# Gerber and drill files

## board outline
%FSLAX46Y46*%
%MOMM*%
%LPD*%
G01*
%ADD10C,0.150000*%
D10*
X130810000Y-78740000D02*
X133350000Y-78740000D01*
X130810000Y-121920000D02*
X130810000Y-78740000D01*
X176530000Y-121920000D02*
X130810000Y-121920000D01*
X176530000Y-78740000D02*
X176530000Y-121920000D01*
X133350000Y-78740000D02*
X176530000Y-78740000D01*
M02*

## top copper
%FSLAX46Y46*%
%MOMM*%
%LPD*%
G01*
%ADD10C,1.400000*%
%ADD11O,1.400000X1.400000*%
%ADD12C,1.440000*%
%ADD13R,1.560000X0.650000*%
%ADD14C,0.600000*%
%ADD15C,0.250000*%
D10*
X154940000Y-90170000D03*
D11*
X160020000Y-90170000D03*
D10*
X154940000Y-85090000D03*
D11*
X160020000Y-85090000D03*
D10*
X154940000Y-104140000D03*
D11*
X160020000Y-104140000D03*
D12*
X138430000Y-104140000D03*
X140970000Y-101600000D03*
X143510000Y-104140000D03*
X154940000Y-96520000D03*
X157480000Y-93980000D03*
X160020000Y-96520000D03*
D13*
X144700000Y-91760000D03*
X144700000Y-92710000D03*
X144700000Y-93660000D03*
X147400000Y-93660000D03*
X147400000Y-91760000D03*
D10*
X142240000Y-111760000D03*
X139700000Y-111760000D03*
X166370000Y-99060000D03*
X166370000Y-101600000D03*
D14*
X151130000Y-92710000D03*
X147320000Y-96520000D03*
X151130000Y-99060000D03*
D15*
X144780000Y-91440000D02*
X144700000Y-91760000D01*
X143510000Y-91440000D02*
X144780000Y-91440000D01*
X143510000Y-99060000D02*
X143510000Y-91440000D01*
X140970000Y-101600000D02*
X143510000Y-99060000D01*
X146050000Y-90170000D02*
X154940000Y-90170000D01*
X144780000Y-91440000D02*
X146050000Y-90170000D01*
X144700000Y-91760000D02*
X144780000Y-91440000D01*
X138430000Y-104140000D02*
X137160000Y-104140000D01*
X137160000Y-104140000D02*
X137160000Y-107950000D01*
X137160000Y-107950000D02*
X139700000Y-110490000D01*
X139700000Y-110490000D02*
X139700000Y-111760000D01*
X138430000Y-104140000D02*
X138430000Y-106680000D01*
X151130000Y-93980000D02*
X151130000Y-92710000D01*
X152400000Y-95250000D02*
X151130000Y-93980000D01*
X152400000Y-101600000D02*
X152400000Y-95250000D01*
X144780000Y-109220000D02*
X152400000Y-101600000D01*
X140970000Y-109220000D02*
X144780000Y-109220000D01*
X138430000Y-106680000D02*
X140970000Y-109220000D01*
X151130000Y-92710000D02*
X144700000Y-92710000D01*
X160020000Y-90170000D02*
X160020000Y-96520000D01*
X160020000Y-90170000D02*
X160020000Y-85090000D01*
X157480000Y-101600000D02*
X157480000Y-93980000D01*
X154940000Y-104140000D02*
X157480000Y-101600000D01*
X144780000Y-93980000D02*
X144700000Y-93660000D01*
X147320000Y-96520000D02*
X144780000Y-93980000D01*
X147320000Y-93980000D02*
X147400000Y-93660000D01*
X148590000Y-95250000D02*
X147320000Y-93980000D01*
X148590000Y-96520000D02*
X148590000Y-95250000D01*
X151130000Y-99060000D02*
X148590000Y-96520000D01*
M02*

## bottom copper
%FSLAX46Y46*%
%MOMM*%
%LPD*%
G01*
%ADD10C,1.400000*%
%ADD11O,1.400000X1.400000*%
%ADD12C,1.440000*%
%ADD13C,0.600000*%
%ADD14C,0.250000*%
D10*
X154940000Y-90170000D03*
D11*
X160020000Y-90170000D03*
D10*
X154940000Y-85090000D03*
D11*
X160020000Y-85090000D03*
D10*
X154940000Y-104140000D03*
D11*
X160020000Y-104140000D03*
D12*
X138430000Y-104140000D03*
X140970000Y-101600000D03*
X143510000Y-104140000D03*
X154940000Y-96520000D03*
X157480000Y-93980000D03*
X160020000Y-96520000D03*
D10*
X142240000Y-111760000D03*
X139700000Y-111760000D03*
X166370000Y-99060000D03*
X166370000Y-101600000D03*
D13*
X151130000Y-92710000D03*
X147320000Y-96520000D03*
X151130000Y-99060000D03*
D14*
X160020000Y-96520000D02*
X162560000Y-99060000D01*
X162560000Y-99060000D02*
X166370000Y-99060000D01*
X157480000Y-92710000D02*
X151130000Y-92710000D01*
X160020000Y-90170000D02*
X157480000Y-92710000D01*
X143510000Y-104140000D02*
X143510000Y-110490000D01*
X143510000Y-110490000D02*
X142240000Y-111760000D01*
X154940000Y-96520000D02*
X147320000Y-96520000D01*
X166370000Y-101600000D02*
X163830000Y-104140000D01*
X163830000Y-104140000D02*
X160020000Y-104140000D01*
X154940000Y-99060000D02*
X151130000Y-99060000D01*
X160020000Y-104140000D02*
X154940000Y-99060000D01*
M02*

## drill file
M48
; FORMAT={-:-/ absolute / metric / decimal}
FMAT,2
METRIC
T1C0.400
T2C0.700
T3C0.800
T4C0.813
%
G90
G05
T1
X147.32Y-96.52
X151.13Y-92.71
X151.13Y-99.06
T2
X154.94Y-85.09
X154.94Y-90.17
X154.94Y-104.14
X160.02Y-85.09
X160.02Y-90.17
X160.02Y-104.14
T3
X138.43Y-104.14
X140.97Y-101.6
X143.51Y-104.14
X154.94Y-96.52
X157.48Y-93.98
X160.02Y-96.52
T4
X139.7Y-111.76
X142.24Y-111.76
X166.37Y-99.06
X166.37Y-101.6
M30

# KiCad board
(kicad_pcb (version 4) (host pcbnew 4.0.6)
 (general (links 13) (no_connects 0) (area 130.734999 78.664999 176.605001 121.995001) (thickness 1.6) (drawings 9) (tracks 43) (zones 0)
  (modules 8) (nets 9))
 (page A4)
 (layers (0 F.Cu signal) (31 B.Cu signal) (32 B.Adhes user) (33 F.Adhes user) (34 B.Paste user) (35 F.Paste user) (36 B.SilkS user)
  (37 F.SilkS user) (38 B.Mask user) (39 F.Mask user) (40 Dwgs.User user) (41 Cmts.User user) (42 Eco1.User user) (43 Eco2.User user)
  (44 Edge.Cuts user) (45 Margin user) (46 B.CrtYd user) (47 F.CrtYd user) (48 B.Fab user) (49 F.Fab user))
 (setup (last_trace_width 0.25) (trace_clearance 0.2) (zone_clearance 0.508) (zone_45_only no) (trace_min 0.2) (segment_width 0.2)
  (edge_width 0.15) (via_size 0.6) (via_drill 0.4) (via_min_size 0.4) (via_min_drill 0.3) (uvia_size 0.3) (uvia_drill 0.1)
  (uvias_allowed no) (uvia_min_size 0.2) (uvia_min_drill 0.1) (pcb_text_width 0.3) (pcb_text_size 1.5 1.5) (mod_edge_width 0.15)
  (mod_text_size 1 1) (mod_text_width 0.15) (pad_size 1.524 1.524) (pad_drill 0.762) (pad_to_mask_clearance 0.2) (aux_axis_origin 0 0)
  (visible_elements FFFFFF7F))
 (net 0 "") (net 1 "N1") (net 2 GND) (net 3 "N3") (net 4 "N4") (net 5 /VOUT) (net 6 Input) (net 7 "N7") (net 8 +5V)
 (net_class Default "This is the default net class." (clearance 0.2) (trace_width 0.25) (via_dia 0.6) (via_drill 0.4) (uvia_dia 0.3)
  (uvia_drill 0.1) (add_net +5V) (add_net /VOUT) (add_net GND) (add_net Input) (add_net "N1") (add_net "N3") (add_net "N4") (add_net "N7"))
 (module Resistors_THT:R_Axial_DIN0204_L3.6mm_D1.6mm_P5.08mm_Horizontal (layer F.Cu) (at 154.94 90.17)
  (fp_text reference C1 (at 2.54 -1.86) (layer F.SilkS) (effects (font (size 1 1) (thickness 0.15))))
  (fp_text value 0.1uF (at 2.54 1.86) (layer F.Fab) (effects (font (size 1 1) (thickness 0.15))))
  (pad 1 thru_hole circle (at 0 0) (size 1.4 1.4) (drill 0.7) (layers *.Cu *.Mask) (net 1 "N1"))
  (pad 2 thru_hole oval (at 5.08 0) (size 1.4 1.4) (drill 0.7) (layers *.Cu *.Mask) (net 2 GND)))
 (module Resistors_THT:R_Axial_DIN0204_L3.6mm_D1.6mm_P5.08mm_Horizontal (layer F.Cu) (at 154.94 85.09)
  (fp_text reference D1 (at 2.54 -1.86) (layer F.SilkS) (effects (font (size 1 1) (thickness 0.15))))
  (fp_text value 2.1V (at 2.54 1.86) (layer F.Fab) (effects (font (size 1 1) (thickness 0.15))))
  (pad 1 thru_hole circle (at 0 0) (size 1.4 1.4) (drill 0.7) (layers *.Cu *.Mask) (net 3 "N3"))
  (pad 2 thru_hole oval (at 5.08 0) (size 1.4 1.4) (drill 0.7) (layers *.Cu *.Mask) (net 2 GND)))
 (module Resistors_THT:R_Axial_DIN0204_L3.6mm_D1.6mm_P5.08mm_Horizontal (layer F.Cu) (at 154.94 104.14)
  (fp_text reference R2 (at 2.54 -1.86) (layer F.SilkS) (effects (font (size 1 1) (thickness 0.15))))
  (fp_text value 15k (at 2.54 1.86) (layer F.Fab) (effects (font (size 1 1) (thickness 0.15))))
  (pad 1 thru_hole circle (at 0 0) (size 1.4 1.4) (drill 0.7) (layers *.Cu *.Mask) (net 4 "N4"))
  (pad 2 thru_hole oval (at 5.08 0) (size 1.4 1.4) (drill 0.7) (layers *.Cu *.Mask) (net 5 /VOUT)))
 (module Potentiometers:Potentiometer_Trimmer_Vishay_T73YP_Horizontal (layer F.Cu) (at 143.51 104.14 90)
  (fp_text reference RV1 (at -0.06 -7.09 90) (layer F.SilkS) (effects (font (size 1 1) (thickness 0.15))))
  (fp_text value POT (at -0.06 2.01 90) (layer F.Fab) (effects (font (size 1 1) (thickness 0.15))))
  (pad 3 thru_hole circle (at 0 -5.08 90) (size 1.44 1.44) (drill 0.8) (layers *.Cu *.Mask) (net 2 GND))
  (pad 2 thru_hole circle (at 2.54 -2.54 90) (size 1.44 1.44) (drill 0.8) (layers *.Cu *.Mask) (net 1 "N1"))
  (pad 1 thru_hole circle (at 0 0 90) (size 1.44 1.44) (drill 0.8) (layers *.Cu *.Mask) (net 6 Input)))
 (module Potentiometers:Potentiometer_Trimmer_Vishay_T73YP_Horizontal (layer F.Cu) (at 160.02 96.52 90)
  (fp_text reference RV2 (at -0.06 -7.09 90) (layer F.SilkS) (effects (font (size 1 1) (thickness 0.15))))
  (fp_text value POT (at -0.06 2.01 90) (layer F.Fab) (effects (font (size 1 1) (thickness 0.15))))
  (pad 3 thru_hole circle (at 0 -5.08 90) (size 1.44 1.44) (drill 0.8) (layers *.Cu *.Mask) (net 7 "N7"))
  (pad 2 thru_hole circle (at 2.54 -2.54 90) (size 1.44 1.44) (drill 0.8) (layers *.Cu *.Mask) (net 4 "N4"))
  (pad 1 thru_hole circle (at 0 0 90) (size 1.44 1.44) (drill 0.8) (layers *.Cu *.Mask) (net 2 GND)))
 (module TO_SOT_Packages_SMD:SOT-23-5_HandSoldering (layer F.Cu) (at 146.05 92.71)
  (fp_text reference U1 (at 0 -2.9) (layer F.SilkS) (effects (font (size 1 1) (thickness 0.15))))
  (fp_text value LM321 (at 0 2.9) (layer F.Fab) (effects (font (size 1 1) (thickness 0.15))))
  (pad 1 smd rect (at -1.35 -0.95) (size 1.56 0.65) (layers F.Cu F.Paste F.Mask) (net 1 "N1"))
  (pad 2 smd rect (at -1.35 0) (size 1.56 0.65) (layers F.Cu F.Paste F.Mask) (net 2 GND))
  (pad 3 smd rect (at -1.35 0.95) (size 1.56 0.65) (layers F.Cu F.Paste F.Mask) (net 7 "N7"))
  (pad 4 smd rect (at 1.35 0.95) (size 1.56 0.65) (layers F.Cu F.Paste F.Mask) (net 5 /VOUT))
  (pad 5 smd rect (at 1.35 -0.95) (size 1.56 0.65) (layers F.Cu F.Paste F.Mask) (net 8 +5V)))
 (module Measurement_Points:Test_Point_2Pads (layer F.Cu) (at 142.24 111.76 180)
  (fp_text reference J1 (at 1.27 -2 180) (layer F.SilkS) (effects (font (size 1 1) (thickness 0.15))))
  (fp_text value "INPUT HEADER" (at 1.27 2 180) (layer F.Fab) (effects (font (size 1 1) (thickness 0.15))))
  (pad 1 thru_hole circle (at 0 0 180) (size 1.4 1.4) (drill 0.8128) (layers *.Cu *.Mask) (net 6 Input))
  (pad 2 thru_hole circle (at 2.54 0 180) (size 1.4 1.4) (drill 0.8128) (layers *.Cu *.Mask) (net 2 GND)))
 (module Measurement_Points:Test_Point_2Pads (layer F.Cu) (at 166.37 99.06 270)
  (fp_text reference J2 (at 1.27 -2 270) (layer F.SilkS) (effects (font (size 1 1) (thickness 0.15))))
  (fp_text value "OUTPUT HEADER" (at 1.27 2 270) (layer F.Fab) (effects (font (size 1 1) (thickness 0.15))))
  (pad 1 thru_hole circle (at 0 0 270) (size 1.4 1.4) (drill 0.8128) (layers *.Cu *.Mask) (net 2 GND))
  (pad 2 thru_hole circle (at 2.54 0 270) (size 1.4 1.4) (drill 0.8128) (layers *.Cu *.Mask) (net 5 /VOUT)))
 (gr_line (start 130.81 78.74) (end 133.35 78.74) (angle 90) (layer Edge.Cuts) (width 0.15))
 (gr_line (start 130.81 121.92) (end 130.81 78.74) (angle 90) (layer Edge.Cuts) (width 0.15))
 (gr_line (start 176.53 121.92) (end 130.81 121.92) (angle 90) (layer Edge.Cuts) (width 0.15))
 (gr_line (start 176.53 78.74) (end 176.53 121.92) (angle 90) (layer Edge.Cuts) (width 0.15))
 (gr_line (start 133.35 78.74) (end 176.53 78.74) (angle 90) (layer Edge.Cuts) (width 0.15))
 (segment (start 144.78 91.44) (end 144.7 91.76) (width 0.25) (layer F.Cu) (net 1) (status 80000))
 (segment (start 143.51 91.44) (end 144.78 91.44) (width 0.25) (layer F.Cu) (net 1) (status 80000))
 (segment (start 143.51 99.06) (end 143.51 91.44) (width 0.25) (layer F.Cu) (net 1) (status 80000))
 (segment (start 140.97 101.6) (end 143.51 99.06) (width 0.25) (layer F.Cu) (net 1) (status 80000))
 (segment (start 146.05 90.17) (end 154.94 90.17) (width 0.25) (layer F.Cu) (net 1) (status 80000))
 (segment (start 144.78 91.44) (end 146.05 90.17) (width 0.25) (layer F.Cu) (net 1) (status 80000))
 (segment (start 144.7 91.76) (end 144.78 91.44) (width 0.25) (layer F.Cu) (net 1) (status 80000))
 (segment (start 160.02 96.52) (end 162.56 99.06) (width 0.25) (layer B.Cu) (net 2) (status 80000))
 (segment (start 162.56 99.06) (end 166.37 99.06) (width 0.25) (layer B.Cu) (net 2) (status 80000))
 (segment (start 138.43 104.14) (end 137.16 104.14) (width 0.25) (layer F.Cu) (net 2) (status 80000))
 (segment (start 137.16 104.14) (end 137.16 107.95) (width 0.25) (layer F.Cu) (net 2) (status 80000))
 (segment (start 137.16 107.95) (end 139.7 110.49) (width 0.25) (layer F.Cu) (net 2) (status 80000))
 (segment (start 139.7 110.49) (end 139.7 111.76) (width 0.25) (layer F.Cu) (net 2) (status 80000))
 (segment (start 138.43 104.14) (end 138.43 106.68) (width 0.25) (layer F.Cu) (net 2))
 (segment (start 151.13 93.98) (end 151.13 92.71) (width 0.25) (layer F.Cu) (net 2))
 (segment (start 152.4 95.25) (end 151.13 93.98) (width 0.25) (layer F.Cu) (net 2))
 (segment (start 152.4 101.6) (end 152.4 95.25) (width 0.25) (layer F.Cu) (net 2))
 (segment (start 144.78 109.22) (end 152.4 101.6) (width 0.25) (layer F.Cu) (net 2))
 (segment (start 140.97 109.22) (end 144.78 109.22) (width 0.25) (layer F.Cu) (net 2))
 (segment (start 138.43 106.68) (end 140.97 109.22) (width 0.25) (layer F.Cu) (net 2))
 (segment (start 151.13 92.71) (end 144.7 92.71) (width 0.25) (layer F.Cu) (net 2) (status 80000))
 (via (at 151.13 92.71) (size 0.6) (layers F.Cu B.Cu) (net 2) (status 80000))
 (segment (start 157.48 92.71) (end 151.13 92.71) (width 0.25) (layer B.Cu) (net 2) (status 80000))
 (segment (start 160.02 90.17) (end 157.48 92.71) (width 0.25) (layer B.Cu) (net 2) (status 80000))
 (segment (start 160.02 90.17) (end 160.02 96.52) (width 0.25) (layer F.Cu) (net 2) (status 80000))
 (segment (start 160.02 90.17) (end 160.02 85.09) (width 0.25) (layer F.Cu) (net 2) (status 80000))
 (segment (start 157.48 101.6) (end 157.48 93.98) (width 0.25) (layer F.Cu) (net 4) (status 80000))
 (segment (start 154.94 104.14) (end 157.48 101.6) (width 0.25) (layer F.Cu) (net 4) (status 80000))
 (segment (start 143.51 104.14) (end 143.51 110.49) (width 0.25) (layer B.Cu) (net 6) (status 80000))
 (segment (start 143.51 110.49) (end 142.24 111.76) (width 0.25) (layer B.Cu) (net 6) (status 80000))
 (segment (start 144.78 93.98) (end 144.7 93.66) (width 0.25) (layer F.Cu) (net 7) (status 80000))
 (segment (start 147.32 96.52) (end 144.78 93.98) (width 0.25) (layer F.Cu) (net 7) (status 80000))
 (via (at 147.32 96.52) (size 0.6) (layers F.Cu B.Cu) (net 7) (status 80000))
 (segment (start 154.94 96.52) (end 147.32 96.52) (width 0.25) (layer B.Cu) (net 7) (status 80000))
 (segment (start 166.37 101.6) (end 163.83 104.14) (width 0.25) (layer B.Cu) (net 5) (status 80000))
 (segment (start 163.83 104.14) (end 160.02 104.14) (width 0.25) (layer B.Cu) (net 5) (status 80000))
 (segment (start 147.32 93.98) (end 147.4 93.66) (width 0.25) (layer F.Cu) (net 5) (status 80000))
 (segment (start 148.59 95.25) (end 147.32 93.98) (width 0.25) (layer F.Cu) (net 5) (status 80000))
 (segment (start 148.59 96.52) (end 148.59 95.25) (width 0.25) (layer F.Cu) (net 5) (status 80000))
 (segment (start 151.13 99.06) (end 148.59 96.52) (width 0.25) (layer F.Cu) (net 5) (status 80000))
 (via (at 151.13 99.06) (size 0.6) (layers F.Cu B.Cu) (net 5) (status 80000))
 (segment (start 154.94 99.06) (end 151.13 99.06) (width 0.25) (layer B.Cu) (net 5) (status 80000))
 (segment (start 160.02 104.14) (end 154.94 99.06) (width 0.25) (layer B.Cu) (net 5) (status 80000)))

